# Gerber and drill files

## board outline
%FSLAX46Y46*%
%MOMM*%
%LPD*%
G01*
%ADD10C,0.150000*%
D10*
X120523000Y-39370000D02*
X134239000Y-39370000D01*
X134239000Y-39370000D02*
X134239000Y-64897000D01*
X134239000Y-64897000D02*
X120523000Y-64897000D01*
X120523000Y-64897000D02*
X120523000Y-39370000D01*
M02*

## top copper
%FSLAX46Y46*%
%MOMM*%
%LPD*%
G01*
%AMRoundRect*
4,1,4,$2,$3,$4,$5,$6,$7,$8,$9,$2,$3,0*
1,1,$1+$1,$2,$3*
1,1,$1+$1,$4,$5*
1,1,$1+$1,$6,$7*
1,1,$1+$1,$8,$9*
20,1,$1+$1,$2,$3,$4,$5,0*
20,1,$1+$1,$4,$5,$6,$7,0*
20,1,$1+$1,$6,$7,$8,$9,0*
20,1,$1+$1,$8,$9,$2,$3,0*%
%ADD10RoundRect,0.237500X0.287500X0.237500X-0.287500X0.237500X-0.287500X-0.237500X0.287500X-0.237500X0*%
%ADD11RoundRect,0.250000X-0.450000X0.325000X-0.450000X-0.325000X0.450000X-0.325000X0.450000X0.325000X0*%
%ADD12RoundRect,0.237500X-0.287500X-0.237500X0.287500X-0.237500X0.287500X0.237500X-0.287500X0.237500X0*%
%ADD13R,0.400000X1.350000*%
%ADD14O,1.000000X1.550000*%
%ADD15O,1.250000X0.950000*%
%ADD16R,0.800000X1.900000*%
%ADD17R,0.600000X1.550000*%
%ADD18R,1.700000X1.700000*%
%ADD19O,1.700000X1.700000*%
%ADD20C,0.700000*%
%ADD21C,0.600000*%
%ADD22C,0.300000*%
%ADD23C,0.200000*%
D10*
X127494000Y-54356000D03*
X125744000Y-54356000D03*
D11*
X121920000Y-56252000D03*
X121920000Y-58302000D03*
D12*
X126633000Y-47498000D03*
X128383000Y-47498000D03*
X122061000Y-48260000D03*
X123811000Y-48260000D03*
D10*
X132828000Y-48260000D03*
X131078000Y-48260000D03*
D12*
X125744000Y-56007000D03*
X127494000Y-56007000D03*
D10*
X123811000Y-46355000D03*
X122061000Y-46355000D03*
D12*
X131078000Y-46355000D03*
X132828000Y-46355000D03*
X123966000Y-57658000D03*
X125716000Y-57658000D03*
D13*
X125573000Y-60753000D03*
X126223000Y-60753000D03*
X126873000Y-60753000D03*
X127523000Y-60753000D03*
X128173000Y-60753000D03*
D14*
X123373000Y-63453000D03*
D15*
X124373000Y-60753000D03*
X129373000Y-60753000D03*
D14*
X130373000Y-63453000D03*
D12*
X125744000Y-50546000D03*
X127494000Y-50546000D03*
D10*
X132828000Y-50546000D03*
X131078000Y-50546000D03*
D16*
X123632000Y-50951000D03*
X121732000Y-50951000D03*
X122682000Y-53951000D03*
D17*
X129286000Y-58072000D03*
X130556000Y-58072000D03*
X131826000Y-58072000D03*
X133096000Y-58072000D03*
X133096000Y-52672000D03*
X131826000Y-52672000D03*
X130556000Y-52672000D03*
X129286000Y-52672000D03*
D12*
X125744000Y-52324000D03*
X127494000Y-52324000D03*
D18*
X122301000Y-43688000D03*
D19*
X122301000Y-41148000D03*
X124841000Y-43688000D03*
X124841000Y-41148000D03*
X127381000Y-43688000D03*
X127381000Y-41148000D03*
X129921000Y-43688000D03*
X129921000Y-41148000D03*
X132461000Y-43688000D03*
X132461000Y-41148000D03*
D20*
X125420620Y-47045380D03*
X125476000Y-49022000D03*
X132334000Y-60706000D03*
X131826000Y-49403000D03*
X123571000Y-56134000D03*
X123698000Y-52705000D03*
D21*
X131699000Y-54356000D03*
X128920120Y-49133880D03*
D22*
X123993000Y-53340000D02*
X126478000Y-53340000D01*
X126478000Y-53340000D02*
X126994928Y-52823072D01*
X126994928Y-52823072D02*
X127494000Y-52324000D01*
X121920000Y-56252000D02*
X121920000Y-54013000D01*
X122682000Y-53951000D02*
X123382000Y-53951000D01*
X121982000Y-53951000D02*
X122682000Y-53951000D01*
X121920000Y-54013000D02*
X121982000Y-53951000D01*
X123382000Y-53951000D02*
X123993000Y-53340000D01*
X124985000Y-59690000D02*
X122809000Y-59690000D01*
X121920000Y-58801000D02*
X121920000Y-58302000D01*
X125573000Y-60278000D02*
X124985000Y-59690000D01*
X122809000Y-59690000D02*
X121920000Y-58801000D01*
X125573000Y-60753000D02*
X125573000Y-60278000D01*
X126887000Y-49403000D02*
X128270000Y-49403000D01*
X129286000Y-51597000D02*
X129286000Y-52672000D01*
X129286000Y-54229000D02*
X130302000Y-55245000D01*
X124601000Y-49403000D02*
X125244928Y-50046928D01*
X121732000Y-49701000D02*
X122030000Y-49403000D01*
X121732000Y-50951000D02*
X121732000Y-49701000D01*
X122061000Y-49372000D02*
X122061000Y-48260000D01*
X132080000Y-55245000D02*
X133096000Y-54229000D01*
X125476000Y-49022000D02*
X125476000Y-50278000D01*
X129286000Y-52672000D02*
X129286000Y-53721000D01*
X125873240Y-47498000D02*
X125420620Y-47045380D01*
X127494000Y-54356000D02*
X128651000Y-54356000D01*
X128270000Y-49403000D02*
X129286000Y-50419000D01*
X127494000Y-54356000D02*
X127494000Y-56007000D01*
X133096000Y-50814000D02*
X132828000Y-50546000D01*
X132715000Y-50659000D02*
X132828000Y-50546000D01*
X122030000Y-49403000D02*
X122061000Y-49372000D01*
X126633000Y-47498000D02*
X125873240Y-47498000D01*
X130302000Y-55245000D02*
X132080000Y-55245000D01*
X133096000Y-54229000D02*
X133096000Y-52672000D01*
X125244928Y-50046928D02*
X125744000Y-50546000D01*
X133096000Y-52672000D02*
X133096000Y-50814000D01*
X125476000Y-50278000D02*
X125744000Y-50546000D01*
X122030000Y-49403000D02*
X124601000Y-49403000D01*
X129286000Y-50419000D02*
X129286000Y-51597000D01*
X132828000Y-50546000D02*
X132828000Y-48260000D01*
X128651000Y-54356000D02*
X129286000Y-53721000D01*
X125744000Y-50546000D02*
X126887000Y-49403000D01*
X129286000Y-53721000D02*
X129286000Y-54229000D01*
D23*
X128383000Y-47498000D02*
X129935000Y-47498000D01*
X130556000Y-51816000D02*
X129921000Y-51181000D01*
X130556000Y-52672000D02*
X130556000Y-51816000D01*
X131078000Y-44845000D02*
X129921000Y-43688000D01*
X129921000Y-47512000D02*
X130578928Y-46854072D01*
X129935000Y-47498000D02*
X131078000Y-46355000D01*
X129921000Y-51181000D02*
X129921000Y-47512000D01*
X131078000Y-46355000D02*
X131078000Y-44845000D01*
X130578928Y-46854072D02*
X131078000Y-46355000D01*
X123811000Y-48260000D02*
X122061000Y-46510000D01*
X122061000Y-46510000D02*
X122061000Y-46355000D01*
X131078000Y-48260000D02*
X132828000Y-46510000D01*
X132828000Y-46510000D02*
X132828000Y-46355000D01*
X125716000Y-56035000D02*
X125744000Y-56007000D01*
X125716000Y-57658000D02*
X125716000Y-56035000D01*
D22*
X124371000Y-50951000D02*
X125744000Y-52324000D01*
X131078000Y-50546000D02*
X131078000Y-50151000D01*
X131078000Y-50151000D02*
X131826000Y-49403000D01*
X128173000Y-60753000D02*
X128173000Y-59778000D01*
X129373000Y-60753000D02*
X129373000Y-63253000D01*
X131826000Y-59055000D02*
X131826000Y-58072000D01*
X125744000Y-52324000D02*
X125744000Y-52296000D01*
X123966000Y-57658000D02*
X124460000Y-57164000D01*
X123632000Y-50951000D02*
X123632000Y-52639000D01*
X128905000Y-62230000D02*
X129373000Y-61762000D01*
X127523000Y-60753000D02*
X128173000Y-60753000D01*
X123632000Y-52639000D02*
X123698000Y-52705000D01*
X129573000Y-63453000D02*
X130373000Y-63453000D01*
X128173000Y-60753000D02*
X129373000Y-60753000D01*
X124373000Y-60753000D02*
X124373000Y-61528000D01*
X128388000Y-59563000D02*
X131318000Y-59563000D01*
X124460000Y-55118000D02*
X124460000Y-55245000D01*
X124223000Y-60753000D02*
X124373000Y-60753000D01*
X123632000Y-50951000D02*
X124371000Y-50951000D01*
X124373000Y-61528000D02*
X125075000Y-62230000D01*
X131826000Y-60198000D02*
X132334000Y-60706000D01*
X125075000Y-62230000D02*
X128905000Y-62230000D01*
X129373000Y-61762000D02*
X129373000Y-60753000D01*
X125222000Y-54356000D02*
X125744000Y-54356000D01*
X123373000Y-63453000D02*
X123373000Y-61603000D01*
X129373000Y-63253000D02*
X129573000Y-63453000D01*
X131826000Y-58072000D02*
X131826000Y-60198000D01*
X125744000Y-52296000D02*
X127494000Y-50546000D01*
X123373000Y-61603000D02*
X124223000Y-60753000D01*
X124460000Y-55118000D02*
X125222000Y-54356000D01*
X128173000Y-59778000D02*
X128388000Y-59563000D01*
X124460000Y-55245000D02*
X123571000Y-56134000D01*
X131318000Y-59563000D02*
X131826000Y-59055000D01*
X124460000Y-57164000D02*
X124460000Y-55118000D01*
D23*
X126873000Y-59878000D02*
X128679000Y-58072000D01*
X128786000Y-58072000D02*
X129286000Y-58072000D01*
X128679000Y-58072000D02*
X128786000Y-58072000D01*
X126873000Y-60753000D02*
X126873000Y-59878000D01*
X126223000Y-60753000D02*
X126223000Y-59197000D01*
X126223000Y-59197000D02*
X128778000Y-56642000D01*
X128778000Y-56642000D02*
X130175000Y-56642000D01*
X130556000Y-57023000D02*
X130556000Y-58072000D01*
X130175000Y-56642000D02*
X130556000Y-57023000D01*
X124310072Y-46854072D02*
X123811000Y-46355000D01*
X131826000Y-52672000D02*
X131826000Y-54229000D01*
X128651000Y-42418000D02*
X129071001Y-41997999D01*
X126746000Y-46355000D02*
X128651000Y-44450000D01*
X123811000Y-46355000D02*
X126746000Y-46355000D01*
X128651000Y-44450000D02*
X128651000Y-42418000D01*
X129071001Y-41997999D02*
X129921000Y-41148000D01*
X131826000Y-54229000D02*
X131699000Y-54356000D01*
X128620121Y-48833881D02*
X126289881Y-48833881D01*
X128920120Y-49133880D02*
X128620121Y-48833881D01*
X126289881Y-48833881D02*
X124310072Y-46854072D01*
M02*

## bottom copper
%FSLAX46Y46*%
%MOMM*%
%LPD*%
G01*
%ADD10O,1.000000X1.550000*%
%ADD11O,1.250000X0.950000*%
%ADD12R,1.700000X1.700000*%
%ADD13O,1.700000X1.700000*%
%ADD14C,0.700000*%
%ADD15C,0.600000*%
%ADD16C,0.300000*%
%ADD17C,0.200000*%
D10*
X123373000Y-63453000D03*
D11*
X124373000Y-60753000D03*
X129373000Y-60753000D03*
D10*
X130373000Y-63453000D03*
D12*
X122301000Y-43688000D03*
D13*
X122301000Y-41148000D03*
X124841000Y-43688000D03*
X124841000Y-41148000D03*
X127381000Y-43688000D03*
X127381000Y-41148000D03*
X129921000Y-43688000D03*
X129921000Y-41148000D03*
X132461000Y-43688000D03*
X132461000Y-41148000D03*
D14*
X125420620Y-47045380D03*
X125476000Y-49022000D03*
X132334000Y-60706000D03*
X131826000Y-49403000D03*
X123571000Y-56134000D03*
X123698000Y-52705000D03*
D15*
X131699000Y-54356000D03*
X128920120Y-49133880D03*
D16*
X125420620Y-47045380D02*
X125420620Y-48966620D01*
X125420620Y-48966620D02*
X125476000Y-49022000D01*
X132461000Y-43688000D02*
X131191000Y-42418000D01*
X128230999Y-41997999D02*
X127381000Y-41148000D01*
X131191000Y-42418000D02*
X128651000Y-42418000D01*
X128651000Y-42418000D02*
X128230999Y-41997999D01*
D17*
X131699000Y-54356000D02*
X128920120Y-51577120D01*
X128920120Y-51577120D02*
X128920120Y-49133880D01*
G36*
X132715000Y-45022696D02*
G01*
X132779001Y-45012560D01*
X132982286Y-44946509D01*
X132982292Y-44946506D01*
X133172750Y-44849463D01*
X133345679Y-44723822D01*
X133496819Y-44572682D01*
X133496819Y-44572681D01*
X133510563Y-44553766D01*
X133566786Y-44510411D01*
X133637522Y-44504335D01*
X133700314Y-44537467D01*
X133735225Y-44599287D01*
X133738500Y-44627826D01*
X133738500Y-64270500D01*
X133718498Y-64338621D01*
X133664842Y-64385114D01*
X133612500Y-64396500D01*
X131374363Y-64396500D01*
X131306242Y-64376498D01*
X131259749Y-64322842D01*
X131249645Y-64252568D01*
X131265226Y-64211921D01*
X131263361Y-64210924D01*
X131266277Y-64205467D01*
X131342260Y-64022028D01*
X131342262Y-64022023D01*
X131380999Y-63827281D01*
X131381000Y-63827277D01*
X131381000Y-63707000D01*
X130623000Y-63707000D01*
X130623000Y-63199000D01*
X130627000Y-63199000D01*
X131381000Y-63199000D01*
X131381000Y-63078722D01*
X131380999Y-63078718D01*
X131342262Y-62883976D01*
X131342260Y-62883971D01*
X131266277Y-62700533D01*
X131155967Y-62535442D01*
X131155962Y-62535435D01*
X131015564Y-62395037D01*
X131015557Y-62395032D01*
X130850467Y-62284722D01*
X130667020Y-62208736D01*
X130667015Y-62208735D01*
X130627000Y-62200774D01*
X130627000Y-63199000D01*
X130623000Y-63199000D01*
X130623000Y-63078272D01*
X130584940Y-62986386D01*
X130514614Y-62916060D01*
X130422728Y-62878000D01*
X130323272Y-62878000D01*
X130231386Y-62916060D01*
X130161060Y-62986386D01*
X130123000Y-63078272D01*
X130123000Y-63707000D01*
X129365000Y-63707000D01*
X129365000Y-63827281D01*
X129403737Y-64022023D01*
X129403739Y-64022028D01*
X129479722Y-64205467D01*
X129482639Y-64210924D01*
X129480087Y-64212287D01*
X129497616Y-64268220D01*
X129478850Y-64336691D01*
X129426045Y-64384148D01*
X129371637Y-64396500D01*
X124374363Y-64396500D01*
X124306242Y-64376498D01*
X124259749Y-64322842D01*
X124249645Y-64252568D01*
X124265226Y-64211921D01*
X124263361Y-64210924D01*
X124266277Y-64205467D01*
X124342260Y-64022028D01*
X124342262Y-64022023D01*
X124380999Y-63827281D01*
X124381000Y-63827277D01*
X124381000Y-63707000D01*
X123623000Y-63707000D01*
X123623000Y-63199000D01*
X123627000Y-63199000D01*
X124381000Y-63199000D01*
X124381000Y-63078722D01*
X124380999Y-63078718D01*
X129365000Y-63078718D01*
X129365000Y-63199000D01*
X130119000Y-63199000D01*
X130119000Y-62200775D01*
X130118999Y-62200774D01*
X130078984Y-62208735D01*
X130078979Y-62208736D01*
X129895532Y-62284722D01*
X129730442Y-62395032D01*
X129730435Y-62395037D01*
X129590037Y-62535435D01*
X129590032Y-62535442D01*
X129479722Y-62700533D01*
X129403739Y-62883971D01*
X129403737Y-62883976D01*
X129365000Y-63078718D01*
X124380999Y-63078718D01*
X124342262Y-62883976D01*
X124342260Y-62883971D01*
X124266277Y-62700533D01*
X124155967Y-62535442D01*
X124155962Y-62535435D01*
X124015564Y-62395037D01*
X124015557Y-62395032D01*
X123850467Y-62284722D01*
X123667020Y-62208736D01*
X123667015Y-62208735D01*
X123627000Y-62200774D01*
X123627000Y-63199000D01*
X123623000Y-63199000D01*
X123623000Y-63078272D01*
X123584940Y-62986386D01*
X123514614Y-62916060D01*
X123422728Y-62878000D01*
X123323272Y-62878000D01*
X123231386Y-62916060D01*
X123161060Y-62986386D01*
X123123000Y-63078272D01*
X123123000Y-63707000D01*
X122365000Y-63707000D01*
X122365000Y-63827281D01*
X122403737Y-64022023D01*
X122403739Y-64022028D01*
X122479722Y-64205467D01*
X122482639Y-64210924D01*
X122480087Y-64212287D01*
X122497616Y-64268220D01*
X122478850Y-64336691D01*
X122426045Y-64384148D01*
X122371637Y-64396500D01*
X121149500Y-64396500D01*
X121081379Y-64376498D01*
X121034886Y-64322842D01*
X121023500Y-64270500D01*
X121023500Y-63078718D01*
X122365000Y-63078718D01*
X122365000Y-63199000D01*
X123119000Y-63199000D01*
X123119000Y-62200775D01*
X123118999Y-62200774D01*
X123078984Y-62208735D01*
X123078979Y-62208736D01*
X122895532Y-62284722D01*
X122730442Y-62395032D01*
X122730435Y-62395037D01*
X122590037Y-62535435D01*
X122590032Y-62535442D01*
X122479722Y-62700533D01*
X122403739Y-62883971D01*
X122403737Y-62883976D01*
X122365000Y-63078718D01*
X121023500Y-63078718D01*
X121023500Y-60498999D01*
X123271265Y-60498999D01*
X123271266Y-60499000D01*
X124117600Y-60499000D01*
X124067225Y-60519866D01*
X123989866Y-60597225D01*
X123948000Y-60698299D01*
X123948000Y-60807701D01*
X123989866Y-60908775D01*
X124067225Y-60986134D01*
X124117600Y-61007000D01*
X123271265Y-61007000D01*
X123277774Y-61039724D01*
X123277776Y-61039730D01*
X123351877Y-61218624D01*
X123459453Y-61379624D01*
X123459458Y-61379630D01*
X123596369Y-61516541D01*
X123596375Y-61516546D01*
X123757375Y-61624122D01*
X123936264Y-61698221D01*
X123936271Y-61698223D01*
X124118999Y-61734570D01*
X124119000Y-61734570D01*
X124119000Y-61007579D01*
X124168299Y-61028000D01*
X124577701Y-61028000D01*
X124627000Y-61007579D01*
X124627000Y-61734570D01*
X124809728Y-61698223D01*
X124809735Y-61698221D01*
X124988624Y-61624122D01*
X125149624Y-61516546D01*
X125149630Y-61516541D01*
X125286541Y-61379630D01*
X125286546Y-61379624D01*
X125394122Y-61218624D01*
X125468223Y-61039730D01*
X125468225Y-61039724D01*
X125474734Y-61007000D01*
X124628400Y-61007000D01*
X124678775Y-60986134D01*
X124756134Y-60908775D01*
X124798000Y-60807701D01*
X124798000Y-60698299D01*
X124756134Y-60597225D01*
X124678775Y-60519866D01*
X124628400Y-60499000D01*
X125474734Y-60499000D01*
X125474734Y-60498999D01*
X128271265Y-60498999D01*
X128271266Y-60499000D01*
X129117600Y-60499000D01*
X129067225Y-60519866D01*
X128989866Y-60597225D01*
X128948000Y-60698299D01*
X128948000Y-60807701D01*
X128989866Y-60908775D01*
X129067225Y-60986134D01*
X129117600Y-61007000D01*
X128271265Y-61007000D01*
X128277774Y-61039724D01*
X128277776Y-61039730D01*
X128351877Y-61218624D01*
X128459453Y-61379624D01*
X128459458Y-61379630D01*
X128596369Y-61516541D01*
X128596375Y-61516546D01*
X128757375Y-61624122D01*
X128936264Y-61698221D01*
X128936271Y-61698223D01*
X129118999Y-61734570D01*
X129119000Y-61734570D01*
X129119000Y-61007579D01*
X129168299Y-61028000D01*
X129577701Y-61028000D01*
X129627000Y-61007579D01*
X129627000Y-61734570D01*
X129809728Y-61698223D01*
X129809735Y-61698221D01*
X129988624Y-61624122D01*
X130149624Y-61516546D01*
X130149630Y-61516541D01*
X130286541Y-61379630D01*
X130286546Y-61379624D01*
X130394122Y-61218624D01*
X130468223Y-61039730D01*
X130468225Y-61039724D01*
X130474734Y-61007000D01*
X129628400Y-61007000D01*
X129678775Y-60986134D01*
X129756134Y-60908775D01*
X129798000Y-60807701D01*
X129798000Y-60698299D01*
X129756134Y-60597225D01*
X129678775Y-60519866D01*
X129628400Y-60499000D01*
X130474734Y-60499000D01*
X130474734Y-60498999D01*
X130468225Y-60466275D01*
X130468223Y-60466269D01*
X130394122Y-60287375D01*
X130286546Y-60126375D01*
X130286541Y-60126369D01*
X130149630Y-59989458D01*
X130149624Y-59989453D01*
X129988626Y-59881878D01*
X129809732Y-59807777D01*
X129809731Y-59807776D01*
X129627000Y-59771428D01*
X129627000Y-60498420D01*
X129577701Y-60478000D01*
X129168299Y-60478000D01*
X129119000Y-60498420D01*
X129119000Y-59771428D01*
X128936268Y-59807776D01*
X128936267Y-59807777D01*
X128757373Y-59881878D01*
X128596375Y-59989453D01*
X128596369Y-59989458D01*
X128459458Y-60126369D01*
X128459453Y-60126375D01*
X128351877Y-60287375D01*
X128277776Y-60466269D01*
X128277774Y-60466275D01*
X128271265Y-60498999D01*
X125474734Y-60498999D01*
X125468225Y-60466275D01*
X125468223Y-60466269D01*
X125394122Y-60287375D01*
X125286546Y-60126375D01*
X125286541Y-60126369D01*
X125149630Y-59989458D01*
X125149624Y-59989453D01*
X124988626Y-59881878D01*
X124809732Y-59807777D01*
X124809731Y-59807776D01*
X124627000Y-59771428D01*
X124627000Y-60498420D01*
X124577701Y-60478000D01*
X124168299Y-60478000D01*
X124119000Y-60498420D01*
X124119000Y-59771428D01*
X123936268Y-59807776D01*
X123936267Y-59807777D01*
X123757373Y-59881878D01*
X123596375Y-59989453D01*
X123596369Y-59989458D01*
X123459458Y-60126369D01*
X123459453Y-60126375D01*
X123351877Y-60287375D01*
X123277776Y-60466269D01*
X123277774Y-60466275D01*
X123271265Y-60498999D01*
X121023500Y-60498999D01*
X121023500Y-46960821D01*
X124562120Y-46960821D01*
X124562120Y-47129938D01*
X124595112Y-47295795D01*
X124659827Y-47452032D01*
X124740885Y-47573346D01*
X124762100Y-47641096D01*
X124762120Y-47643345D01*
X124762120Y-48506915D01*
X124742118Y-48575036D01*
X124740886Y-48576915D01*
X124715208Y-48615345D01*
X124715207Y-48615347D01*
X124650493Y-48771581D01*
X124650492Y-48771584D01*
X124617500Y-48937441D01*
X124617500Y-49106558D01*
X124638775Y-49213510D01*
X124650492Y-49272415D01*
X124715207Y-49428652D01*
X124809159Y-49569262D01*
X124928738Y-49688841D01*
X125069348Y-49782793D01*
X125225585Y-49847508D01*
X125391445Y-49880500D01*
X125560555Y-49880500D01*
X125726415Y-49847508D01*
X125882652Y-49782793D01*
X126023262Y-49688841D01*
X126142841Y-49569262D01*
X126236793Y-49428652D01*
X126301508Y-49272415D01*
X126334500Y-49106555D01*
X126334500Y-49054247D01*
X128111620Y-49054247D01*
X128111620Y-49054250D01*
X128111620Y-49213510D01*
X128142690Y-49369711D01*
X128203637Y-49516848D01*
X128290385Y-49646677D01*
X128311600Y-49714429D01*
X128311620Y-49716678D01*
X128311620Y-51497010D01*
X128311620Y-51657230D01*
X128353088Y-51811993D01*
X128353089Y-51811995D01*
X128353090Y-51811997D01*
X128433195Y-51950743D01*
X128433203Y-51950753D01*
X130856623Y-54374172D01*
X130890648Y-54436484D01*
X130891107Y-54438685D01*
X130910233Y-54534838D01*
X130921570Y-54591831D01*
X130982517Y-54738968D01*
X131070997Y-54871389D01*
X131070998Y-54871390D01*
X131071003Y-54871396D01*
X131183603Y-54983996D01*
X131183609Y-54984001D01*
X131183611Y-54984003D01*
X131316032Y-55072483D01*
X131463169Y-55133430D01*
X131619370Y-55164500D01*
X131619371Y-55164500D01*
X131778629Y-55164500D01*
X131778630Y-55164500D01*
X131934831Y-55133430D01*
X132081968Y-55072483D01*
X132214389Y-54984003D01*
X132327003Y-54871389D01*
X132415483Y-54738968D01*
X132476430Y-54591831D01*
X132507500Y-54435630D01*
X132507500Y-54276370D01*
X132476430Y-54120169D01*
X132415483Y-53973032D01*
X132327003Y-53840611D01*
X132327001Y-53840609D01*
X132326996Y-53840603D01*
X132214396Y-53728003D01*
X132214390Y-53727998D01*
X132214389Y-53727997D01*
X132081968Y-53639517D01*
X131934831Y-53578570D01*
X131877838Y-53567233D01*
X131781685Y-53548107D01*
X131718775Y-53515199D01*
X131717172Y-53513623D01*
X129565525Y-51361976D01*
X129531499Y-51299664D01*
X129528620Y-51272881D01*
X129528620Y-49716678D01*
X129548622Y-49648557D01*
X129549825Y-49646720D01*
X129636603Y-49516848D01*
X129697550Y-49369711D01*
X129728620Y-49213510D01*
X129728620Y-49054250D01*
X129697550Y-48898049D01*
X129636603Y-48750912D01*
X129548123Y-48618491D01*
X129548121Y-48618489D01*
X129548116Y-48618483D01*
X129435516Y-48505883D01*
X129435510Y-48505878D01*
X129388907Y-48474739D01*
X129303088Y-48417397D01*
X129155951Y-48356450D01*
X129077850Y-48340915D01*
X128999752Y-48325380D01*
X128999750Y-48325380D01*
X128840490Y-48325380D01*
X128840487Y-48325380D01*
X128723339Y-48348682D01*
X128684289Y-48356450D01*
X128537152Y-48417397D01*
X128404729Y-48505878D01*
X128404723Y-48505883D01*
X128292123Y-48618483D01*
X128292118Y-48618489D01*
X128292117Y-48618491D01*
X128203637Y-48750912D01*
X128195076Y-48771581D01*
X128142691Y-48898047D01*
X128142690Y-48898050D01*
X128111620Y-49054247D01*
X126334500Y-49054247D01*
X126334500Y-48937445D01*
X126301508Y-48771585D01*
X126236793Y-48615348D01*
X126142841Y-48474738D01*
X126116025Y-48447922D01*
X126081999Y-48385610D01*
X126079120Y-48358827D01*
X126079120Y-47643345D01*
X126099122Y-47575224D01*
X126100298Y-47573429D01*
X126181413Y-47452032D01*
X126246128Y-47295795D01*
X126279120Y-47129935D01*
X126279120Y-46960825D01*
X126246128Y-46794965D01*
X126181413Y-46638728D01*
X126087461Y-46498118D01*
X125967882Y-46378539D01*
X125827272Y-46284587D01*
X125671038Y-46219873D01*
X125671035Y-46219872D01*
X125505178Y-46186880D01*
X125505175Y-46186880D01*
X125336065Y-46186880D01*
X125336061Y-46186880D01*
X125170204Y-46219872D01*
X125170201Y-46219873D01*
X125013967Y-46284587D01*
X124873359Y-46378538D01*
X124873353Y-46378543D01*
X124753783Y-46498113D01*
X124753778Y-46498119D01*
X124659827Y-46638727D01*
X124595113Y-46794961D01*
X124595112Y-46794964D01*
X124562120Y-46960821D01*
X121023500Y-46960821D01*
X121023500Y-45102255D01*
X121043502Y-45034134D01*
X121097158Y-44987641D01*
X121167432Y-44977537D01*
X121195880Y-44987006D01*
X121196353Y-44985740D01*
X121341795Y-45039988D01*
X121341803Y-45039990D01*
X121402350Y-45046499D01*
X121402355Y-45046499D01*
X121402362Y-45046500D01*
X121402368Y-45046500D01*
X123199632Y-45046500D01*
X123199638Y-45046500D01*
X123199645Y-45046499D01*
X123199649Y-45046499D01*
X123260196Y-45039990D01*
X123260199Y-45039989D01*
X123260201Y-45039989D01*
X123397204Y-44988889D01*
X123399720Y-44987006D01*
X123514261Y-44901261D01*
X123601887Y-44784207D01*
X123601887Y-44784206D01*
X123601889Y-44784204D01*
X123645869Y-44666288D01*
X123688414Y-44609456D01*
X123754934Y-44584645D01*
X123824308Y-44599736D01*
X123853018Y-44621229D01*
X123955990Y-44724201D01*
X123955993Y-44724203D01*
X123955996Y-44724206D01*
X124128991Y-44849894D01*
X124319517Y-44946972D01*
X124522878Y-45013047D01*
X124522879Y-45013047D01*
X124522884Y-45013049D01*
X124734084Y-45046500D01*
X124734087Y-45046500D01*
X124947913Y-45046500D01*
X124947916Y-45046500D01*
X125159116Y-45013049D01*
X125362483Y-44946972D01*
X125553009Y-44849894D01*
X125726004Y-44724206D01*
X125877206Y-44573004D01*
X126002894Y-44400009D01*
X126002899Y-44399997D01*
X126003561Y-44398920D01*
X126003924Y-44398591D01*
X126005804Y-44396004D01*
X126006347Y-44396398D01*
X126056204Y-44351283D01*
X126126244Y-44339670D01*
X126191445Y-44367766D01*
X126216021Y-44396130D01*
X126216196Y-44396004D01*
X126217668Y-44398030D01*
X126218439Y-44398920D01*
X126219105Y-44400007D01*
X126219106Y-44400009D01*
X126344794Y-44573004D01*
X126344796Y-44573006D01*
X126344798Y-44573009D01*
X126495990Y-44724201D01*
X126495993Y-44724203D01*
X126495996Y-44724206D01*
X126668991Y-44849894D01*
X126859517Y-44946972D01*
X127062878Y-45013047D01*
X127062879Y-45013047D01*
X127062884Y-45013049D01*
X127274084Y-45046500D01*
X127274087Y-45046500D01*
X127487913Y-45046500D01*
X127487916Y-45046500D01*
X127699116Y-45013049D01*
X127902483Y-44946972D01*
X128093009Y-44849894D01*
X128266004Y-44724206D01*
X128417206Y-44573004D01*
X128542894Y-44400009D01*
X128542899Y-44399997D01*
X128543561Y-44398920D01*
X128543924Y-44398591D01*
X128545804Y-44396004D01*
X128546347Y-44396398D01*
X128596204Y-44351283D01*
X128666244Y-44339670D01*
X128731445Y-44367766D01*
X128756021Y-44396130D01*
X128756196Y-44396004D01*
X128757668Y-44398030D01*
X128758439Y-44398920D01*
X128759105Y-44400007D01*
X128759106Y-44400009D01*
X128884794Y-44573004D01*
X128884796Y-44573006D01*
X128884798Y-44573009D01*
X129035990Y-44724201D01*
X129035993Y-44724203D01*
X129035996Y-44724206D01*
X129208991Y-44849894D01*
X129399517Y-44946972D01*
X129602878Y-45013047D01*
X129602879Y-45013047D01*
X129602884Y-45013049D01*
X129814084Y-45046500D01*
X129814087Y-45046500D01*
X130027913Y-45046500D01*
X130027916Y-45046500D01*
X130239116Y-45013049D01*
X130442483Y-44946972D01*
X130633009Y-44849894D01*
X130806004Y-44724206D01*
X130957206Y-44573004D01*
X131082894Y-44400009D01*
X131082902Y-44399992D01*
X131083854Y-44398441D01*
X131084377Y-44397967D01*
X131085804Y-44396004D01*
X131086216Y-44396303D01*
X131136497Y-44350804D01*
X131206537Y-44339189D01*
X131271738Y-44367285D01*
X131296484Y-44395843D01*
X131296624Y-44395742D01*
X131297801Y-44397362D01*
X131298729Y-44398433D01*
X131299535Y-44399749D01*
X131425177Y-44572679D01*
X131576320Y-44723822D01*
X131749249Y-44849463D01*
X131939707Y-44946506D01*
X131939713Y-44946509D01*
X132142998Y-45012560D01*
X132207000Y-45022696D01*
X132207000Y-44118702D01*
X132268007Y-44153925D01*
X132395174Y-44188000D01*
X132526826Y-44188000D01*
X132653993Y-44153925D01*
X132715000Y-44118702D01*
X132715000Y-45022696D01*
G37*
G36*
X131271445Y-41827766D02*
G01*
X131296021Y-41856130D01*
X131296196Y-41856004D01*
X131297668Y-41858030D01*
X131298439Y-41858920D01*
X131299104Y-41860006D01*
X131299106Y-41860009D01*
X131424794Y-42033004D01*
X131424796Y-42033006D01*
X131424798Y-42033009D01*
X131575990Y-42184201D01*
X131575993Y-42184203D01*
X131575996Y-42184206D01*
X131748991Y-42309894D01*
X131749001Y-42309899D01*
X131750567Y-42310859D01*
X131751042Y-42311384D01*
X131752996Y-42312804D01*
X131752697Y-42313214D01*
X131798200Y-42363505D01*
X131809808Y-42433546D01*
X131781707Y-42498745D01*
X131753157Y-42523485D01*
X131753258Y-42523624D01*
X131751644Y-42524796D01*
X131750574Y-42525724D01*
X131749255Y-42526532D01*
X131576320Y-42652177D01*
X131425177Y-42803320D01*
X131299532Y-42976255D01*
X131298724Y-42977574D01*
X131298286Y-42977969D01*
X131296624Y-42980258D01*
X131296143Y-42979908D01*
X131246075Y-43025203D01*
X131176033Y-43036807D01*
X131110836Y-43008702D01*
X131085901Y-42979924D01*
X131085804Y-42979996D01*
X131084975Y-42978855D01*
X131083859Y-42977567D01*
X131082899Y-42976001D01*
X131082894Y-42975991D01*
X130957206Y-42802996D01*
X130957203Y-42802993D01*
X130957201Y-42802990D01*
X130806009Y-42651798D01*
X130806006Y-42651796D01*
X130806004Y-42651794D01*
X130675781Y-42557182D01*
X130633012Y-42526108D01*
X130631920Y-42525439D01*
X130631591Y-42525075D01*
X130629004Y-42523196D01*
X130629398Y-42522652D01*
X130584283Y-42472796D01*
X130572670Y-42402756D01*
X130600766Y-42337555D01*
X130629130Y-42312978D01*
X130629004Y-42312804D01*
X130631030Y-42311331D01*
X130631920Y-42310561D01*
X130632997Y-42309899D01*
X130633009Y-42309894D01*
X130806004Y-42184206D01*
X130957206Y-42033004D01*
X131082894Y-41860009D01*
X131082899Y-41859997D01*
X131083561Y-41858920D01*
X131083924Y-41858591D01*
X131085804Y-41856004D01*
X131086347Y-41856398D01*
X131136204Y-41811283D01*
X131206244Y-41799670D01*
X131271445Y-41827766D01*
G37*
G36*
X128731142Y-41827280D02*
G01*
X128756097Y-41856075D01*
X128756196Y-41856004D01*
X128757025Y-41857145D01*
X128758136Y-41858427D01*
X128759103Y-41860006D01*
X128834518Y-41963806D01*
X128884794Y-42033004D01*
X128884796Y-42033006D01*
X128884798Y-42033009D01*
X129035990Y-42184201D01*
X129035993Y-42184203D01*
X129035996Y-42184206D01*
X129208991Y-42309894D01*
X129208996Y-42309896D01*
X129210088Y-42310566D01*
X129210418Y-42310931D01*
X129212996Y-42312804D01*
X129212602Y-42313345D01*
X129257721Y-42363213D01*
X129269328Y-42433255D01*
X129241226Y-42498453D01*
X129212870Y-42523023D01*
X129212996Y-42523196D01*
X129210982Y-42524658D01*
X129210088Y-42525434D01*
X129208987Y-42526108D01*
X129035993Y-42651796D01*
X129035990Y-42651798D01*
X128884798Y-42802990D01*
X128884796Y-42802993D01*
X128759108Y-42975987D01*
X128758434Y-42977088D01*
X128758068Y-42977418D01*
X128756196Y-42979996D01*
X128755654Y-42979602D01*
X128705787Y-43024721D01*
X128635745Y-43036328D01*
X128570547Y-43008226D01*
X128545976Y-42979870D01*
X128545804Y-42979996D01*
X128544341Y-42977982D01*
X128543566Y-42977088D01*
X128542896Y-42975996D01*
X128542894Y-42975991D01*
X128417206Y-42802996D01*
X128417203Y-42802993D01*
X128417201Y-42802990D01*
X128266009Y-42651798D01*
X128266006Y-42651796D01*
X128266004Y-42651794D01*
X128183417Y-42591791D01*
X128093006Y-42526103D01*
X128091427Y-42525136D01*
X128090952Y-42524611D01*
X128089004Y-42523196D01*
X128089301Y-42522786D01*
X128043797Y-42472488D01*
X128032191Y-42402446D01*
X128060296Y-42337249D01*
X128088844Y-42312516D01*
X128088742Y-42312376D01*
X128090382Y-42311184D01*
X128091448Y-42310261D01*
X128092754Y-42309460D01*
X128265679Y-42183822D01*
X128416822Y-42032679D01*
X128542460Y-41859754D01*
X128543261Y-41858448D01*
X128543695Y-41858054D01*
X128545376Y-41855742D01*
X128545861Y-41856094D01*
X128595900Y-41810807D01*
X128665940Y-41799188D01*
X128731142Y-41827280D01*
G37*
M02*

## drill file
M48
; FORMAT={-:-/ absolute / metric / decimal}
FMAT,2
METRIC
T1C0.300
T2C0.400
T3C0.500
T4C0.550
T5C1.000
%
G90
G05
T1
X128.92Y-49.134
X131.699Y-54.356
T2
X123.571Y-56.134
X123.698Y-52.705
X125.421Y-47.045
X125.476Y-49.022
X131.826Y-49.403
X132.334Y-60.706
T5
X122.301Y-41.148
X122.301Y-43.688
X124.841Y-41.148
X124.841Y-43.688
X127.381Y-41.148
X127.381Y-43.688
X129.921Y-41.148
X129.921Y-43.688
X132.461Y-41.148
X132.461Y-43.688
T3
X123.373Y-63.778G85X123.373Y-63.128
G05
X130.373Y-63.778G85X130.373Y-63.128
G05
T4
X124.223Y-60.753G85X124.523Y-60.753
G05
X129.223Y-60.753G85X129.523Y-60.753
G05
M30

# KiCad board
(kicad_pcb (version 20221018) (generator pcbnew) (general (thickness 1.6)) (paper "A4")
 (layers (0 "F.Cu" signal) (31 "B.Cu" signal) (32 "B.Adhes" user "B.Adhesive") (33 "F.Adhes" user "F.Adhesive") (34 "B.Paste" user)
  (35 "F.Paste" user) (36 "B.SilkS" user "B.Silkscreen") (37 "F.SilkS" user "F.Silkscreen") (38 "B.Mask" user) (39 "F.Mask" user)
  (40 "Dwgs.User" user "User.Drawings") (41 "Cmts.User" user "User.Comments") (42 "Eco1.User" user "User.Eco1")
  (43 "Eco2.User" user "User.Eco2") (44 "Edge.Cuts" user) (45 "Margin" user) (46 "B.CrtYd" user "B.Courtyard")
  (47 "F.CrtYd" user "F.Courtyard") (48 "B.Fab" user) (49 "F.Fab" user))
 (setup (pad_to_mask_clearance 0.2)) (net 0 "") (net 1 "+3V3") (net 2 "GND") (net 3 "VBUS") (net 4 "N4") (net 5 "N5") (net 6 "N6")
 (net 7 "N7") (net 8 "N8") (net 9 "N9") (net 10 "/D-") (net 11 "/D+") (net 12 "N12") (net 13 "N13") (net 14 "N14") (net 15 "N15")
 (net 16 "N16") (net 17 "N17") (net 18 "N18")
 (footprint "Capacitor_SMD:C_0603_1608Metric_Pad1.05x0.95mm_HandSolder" (layer "F.Cu") (at 126.619 54.356 180)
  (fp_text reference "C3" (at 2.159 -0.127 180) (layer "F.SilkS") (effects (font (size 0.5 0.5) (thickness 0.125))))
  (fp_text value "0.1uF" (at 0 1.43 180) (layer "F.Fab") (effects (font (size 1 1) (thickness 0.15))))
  (pad "1" smd roundrect (at -0.875 0 180) (size 1.05 0.95) (layers "F.Cu" "F.Paste" "F.Mask") (roundrect_rratio 0.25) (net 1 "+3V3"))
  (pad "2" smd roundrect (at 0.875 0 180) (size 1.05 0.95) (layers "F.Cu" "F.Paste" "F.Mask") (roundrect_rratio 0.25) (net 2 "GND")))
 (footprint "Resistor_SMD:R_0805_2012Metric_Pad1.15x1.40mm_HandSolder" (layer "F.Cu") (at 121.92 57.277 -90)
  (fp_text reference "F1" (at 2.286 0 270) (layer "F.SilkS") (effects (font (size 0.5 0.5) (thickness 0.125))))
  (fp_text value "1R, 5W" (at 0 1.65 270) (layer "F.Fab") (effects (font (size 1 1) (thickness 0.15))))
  (pad "1" smd roundrect (at -1.025 0 270) (size 1.15 1.4) (layers "F.Cu" "F.Paste" "F.Mask") (roundrect_rratio 0.217391) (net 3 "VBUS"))
  (pad "2" smd roundrect (at 1.025 0 270) (size 1.15 1.4) (layers "F.Cu" "F.Paste" "F.Mask") (roundrect_rratio 0.217391) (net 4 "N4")))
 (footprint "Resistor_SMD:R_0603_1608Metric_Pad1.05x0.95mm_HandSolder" (layer "F.Cu") (at 127.508 47.498)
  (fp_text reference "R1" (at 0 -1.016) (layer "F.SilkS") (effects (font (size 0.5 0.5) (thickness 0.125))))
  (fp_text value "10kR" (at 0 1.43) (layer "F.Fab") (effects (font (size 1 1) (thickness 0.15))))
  (pad "1" smd roundrect (at -0.875 0) (size 1.05 0.95) (layers "F.Cu" "F.Paste" "F.Mask") (roundrect_rratio 0.25) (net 1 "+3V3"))
  (pad "2" smd roundrect (at 0.875 0) (size 1.05 0.95) (layers "F.Cu" "F.Paste" "F.Mask") (roundrect_rratio 0.25) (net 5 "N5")))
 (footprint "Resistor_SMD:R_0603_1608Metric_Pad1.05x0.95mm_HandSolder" (layer "F.Cu") (at 122.936 48.26)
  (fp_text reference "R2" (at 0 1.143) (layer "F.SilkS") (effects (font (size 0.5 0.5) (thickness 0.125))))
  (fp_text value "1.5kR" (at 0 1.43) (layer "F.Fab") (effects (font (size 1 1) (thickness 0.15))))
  (pad "1" smd roundrect (at -0.875 0) (size 1.05 0.95) (layers "F.Cu" "F.Paste" "F.Mask") (roundrect_rratio 0.25) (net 1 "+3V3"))
  (pad "2" smd roundrect (at 0.875 0) (size 1.05 0.95) (layers "F.Cu" "F.Paste" "F.Mask") (roundrect_rratio 0.25) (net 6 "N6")))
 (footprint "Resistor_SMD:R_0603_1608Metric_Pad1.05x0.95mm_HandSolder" (layer "F.Cu") (at 131.953 48.26 180)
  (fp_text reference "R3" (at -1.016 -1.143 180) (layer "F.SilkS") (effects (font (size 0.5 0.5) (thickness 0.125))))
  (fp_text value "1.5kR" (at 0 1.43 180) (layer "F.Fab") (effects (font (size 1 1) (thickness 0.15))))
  (pad "1" smd roundrect (at -0.875 0 180) (size 1.05 0.95) (layers "F.Cu" "F.Paste" "F.Mask") (roundrect_rratio 0.25) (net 1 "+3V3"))
  (pad "2" smd roundrect (at 0.875 0 180) (size 1.05 0.95) (layers "F.Cu" "F.Paste" "F.Mask") (roundrect_rratio 0.25) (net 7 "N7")))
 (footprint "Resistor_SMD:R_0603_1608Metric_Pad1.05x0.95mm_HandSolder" (layer "F.Cu") (at 126.619 56.007)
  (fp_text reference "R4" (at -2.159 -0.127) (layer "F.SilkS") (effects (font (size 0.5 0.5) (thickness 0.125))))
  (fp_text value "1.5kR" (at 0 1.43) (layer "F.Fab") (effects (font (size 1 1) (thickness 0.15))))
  (pad "1" smd roundrect (at -0.875 0) (size 1.05 0.95) (layers "F.Cu" "F.Paste" "F.Mask") (roundrect_rratio 0.25) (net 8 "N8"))
  (pad "2" smd roundrect (at 0.875 0) (size 1.05 0.95) (layers "F.Cu" "F.Paste" "F.Mask") (roundrect_rratio 0.25) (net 1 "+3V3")))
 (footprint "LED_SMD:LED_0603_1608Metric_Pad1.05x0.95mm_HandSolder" (layer "F.Cu") (at 122.936 46.355 180)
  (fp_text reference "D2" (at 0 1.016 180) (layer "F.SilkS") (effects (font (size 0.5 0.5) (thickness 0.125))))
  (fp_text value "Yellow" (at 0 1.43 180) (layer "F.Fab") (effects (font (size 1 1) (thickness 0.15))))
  (pad "1" smd roundrect (at -0.875 0 180) (size 1.05 0.95) (layers "F.Cu" "F.Paste" "F.Mask") (roundrect_rratio 0.25) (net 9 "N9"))
  (pad "2" smd roundrect (at 0.875 0 180) (size 1.05 0.95) (layers "F.Cu" "F.Paste" "F.Mask") (roundrect_rratio 0.25) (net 6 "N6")))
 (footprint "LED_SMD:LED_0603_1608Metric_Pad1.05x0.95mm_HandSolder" (layer "F.Cu") (at 131.953 46.355)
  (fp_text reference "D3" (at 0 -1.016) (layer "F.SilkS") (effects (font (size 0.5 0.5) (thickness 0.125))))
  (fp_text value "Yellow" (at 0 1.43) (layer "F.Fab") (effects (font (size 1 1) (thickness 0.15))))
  (pad "1" smd roundrect (at -0.875 0) (size 1.05 0.95) (layers "F.Cu" "F.Paste" "F.Mask") (roundrect_rratio 0.25) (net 5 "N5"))
  (pad "2" smd roundrect (at 0.875 0) (size 1.05 0.95) (layers "F.Cu" "F.Paste" "F.Mask") (roundrect_rratio 0.25) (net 7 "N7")))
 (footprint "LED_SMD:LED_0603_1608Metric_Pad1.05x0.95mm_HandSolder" (layer "F.Cu") (at 124.841 57.658)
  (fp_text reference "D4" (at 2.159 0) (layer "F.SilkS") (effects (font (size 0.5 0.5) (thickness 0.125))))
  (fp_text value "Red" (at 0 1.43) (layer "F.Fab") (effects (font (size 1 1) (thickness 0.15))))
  (pad "1" smd roundrect (at -0.875 0) (size 1.05 0.95) (layers "F.Cu" "F.Paste" "F.Mask") (roundrect_rratio 0.25) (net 2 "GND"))
  (pad "2" smd roundrect (at 0.875 0) (size 1.05 0.95) (layers "F.Cu" "F.Paste" "F.Mask") (roundrect_rratio 0.25) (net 8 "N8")))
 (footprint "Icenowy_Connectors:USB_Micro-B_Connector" (layer "F.Cu") (at 126.873 62.103)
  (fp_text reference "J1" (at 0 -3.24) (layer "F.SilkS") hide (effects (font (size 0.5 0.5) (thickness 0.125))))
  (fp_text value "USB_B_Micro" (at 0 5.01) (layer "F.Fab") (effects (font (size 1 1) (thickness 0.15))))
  (pad "1" smd rect (at -1.3 -1.35 90) (size 1.35 0.4) (layers "F.Cu" "F.Paste" "F.Mask") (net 4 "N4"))
  (pad "2" smd rect (at -0.65 -1.35 90) (size 1.35 0.4) (layers "F.Cu" "F.Paste" "F.Mask") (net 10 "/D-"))
  (pad "3" smd rect (at 0 -1.35 90) (size 1.35 0.4) (layers "F.Cu" "F.Paste" "F.Mask") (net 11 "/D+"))
  (pad "4" smd rect (at 0.65 -1.35 90) (size 1.35 0.4) (layers "F.Cu" "F.Paste" "F.Mask") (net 2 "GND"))
  (pad "5" smd rect (at 1.3 -1.35 90) (size 1.35 0.4) (layers "F.Cu" "F.Paste" "F.Mask") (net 2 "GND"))
  (pad "6" thru_hole oval (at -3.5 1.35 90) (size 1.55 1) (drill oval 1.15 0.5) (layers "*.Cu" "*.Mask") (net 2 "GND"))
  (pad "6" thru_hole oval (at -2.5 -1.35 90) (size 0.95 1.25) (drill oval 0.55 0.85) (layers "*.Cu" "*.Mask") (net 2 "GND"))
  (pad "6" thru_hole oval (at 2.5 -1.35 90) (size 0.95 1.25) (drill oval 0.55 0.85) (layers "*.Cu" "*.Mask") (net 2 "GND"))
  (pad "6" thru_hole oval (at 3.5 1.35 90) (size 1.55 1) (drill oval 1.15 0.5) (layers "*.Cu" "*.Mask") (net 2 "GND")))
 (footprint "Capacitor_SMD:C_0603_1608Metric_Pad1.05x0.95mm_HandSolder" (layer "F.Cu") (at 126.619 50.546)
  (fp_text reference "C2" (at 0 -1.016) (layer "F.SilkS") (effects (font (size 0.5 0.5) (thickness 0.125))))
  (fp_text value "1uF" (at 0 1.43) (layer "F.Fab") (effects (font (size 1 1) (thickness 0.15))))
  (pad "1" smd roundrect (at -0.875 0) (size 1.05 0.95) (layers "F.Cu" "F.Paste" "F.Mask") (roundrect_rratio 0.25) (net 1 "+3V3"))
  (pad "2" smd roundrect (at 0.875 0) (size 1.05 0.95) (layers "F.Cu" "F.Paste" "F.Mask") (roundrect_rratio 0.25) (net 2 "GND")))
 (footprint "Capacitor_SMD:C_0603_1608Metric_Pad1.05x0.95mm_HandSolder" (layer "F.Cu") (at 131.953 50.546 180)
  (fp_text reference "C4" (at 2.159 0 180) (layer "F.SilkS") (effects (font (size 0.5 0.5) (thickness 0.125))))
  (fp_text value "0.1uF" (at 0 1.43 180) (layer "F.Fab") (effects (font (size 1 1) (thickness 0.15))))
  (pad "1" smd roundrect (at -0.875 0 180) (size 1.05 0.95) (layers "F.Cu" "F.Paste" "F.Mask") (roundrect_rratio 0.25) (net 1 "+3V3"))
  (pad "2" smd roundrect (at 0.875 0 180) (size 1.05 0.95) (layers "F.Cu" "F.Paste" "F.Mask") (roundrect_rratio 0.25) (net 2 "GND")))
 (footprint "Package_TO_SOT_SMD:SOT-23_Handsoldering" (layer "F.Cu") (at 122.682 52.451 -90)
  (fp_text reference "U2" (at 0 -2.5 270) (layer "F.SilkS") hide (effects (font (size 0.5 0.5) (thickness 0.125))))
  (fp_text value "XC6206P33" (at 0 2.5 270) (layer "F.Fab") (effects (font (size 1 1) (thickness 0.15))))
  (pad "1" smd rect (at -1.5 -0.95 270) (size 1.9 0.8) (layers "F.Cu" "F.Paste" "F.Mask") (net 2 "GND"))
  (pad "2" smd rect (at -1.5 0.95 270) (size 1.9 0.8) (layers "F.Cu" "F.Paste" "F.Mask") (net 1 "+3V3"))
  (pad "3" smd rect (at 1.5 0 270) (size 1.9 0.8) (layers "F.Cu" "F.Paste" "F.Mask") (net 3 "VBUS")))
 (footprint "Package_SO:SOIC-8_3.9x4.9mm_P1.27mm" (layer "F.Cu") (at 131.191 55.372 90)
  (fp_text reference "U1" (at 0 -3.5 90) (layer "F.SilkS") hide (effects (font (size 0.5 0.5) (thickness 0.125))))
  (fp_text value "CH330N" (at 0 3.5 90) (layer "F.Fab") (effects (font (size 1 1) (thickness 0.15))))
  (pad "1" smd rect (at -2.7 -1.905 90) (size 1.55 0.6) (layers "F.Cu" "F.Paste" "F.Mask") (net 11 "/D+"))
  (pad "2" smd rect (at -2.7 -0.635 90) (size 1.55 0.6) (layers "F.Cu" "F.Paste" "F.Mask") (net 10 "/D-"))
  (pad "3" smd rect (at -2.7 0.635 90) (size 1.55 0.6) (layers "F.Cu" "F.Paste" "F.Mask") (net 2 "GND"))
  (pad "4" smd rect (at -2.7 1.905 90) (size 1.55 0.6) (layers "F.Cu" "F.Paste" "F.Mask") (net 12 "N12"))
  (pad "5" smd rect (at 2.7 1.905 90) (size 1.55 0.6) (layers "F.Cu" "F.Paste" "F.Mask") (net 1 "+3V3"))
  (pad "6" smd rect (at 2.7 0.635 90) (size 1.55 0.6) (layers "F.Cu" "F.Paste" "F.Mask") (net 9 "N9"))
  (pad "7" smd rect (at 2.7 -0.635 90) (size 1.55 0.6) (layers "F.Cu" "F.Paste" "F.Mask") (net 5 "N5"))
  (pad "8" smd rect (at 2.7 -1.905 90) (size 1.55 0.6) (layers "F.Cu" "F.Paste" "F.Mask") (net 1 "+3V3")))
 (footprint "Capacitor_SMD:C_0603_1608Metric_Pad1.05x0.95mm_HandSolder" (layer "F.Cu") (at 126.619 52.324)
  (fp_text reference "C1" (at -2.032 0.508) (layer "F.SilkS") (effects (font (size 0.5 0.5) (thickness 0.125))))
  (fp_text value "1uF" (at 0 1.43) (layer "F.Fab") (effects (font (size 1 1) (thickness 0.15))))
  (pad "1" smd roundrect (at -0.875 0) (size 1.05 0.95) (layers "F.Cu" "F.Paste" "F.Mask") (roundrect_rratio 0.25) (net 2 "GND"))
  (pad "2" smd roundrect (at 0.875 0) (size 1.05 0.95) (layers "F.Cu" "F.Paste" "F.Mask") (roundrect_rratio 0.25) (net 3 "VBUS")))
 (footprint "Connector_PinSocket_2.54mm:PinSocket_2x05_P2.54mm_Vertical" (layer "B.Cu") (at 122.301 43.688 -90)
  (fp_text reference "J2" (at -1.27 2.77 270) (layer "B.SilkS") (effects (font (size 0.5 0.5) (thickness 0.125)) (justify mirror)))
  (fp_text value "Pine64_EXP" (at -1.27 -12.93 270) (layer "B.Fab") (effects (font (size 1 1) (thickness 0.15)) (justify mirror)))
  (pad "1" thru_hole rect (at 0 0 270) (size 1.7 1.7) (drill 1) (layers "*.Cu" "*.Mask") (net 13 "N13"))
  (pad "2" thru_hole oval (at -2.54 0 270) (size 1.7 1.7) (drill 1) (layers "*.Cu" "*.Mask") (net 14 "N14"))
  (pad "3" thru_hole oval (at 0 -2.54 270) (size 1.7 1.7) (drill 1) (layers "*.Cu" "*.Mask") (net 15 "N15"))
  (pad "4" thru_hole oval (at -2.54 -2.54 270) (size 1.7 1.7) (drill 1) (layers "*.Cu" "*.Mask") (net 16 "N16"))
  (pad "5" thru_hole oval (at 0 -5.08 270) (size 1.7 1.7) (drill 1) (layers "*.Cu" "*.Mask") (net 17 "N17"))
  (pad "6" thru_hole oval (at -2.54 -5.08 270) (size 1.7 1.7) (drill 1) (layers "*.Cu" "*.Mask") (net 2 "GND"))
  (pad "7" thru_hole oval (at 0 -7.62 270) (size 1.7 1.7) (drill 1) (layers "*.Cu" "*.Mask") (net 5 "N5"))
  (pad "8" thru_hole oval (at -2.54 -7.62 270) (size 1.7 1.7) (drill 1) (layers "*.Cu" "*.Mask") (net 9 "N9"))
  (pad "9" thru_hole oval (at 0 -10.16 270) (size 1.7 1.7) (drill 1) (layers "*.Cu" "*.Mask") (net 2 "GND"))
  (pad "10" thru_hole oval (at -2.54 -10.16 270) (size 1.7 1.7) (drill 1) (layers "*.Cu" "*.Mask") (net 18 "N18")))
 (gr_line (start 120.523 39.37) (end 134.239 39.37) (stroke (width 0.15) (type solid)) (layer "Edge.Cuts"))
 (gr_line (start 134.239 39.37) (end 134.239 64.897) (stroke (width 0.15) (type solid)) (layer "Edge.Cuts"))
 (gr_line (start 134.239 64.897) (end 120.523 64.897) (stroke (width 0.15) (type solid)) (layer "Edge.Cuts"))
 (gr_line (start 120.523 64.897) (end 120.523 39.37) (stroke (width 0.15) (type solid)) (layer "Edge.Cuts"))
 (segment (start 123.993 53.34) (end 126.478 53.34) (width 0.3) (layer "F.Cu") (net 3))
 (segment (start 126.478 53.34) (end 126.994928 52.823072) (width 0.3) (layer "F.Cu") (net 3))
 (segment (start 126.994928 52.823072) (end 127.494 52.324) (width 0.3) (layer "F.Cu") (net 3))
 (segment (start 121.92 56.252) (end 121.92 54.013) (width 0.3) (layer "F.Cu") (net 3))
 (segment (start 122.682 53.951) (end 123.382 53.951) (width 0.3) (layer "F.Cu") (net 3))
 (segment (start 121.982 53.951) (end 122.682 53.951) (width 0.3) (layer "F.Cu") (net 3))
 (segment (start 121.92 54.013) (end 121.982 53.951) (width 0.3) (layer "F.Cu") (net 3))
 (segment (start 123.382 53.951) (end 123.993 53.34) (width 0.3) (layer "F.Cu") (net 3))
 (segment (start 124.985 59.69) (end 122.809 59.69) (width 0.3) (layer "F.Cu") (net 4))
 (segment (start 121.92 58.801) (end 121.92 58.302) (width 0.3) (layer "F.Cu") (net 4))
 (segment (start 125.573 60.278) (end 124.985 59.69) (width 0.3) (layer "F.Cu") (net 4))
 (segment (start 122.809 59.69) (end 121.92 58.801) (width 0.3) (layer "F.Cu") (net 4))
 (segment (start 125.573 60.753) (end 125.573 60.278) (width 0.3) (layer "F.Cu") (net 4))
 (segment (start 126.887 49.403) (end 128.27 49.403) (width 0.3) (layer "F.Cu") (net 1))
 (segment (start 129.286 51.597) (end 129.286 52.672) (width 0.3) (layer "F.Cu") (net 1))
 (segment (start 129.286 54.229) (end 130.302 55.245) (width 0.3) (layer "F.Cu") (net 1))
 (segment (start 124.601 49.403) (end 125.244928 50.046928) (width 0.3) (layer "F.Cu") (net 1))
 (segment (start 121.732 49.701) (end 122.03 49.403) (width 0.3) (layer "F.Cu") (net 1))
 (segment (start 121.732 50.951) (end 121.732 49.701) (width 0.3) (layer "F.Cu") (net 1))
 (segment (start 122.061 49.372) (end 122.061 48.26) (width 0.3) (layer "F.Cu") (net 1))
 (segment (start 132.08 55.245) (end 133.096 54.229) (width 0.3) (layer "F.Cu") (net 1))
 (segment (start 125.476 49.022) (end 125.476 50.278) (width 0.3) (layer "F.Cu") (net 1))
 (segment (start 129.286 52.672) (end 129.286 53.721) (width 0.3) (layer "F.Cu") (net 1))
 (segment (start 125.87324 47.498) (end 125.42062 47.04538) (width 0.3) (layer "F.Cu") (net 1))
 (segment (start 127.494 54.356) (end 128.651 54.356) (width 0.3) (layer "F.Cu") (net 1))
 (segment (start 128.27 49.403) (end 129.286 50.419) (width 0.3) (layer "F.Cu") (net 1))
 (segment (start 127.494 54.356) (end 127.494 56.007) (width 0.3) (layer "F.Cu") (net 1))
 (segment (start 133.096 50.814) (end 132.828 50.546) (width 0.3) (layer "F.Cu") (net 1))
 (segment (start 132.715 50.659) (end 132.828 50.546) (width 0.3) (layer "F.Cu") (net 1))
 (segment (start 122.03 49.403) (end 122.061 49.372) (width 0.3) (layer "F.Cu") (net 1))
 (segment (start 126.633 47.498) (end 125.87324 47.498) (width 0.3) (layer "F.Cu") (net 1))
 (segment (start 130.302 55.245) (end 132.08 55.245) (width 0.3) (layer "F.Cu") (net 1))
 (segment (start 133.096 54.229) (end 133.096 52.672) (width 0.3) (layer "F.Cu") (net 1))
 (segment (start 125.244928 50.046928) (end 125.744 50.546) (width 0.3) (layer "F.Cu") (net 1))
 (segment (start 133.096 52.672) (end 133.096 50.814) (width 0.3) (layer "F.Cu") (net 1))
 (segment (start 125.476 50.278) (end 125.744 50.546) (width 0.3) (layer "F.Cu") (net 1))
 (segment (start 122.03 49.403) (end 124.601 49.403) (width 0.3) (layer "F.Cu") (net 1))
 (segment (start 129.286 50.419) (end 129.286 51.597) (width 0.3) (layer "F.Cu") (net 1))
 (segment (start 132.828 50.546) (end 132.828 48.26) (width 0.3) (layer "F.Cu") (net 1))
 (segment (start 128.651 54.356) (end 129.286 53.721) (width 0.3) (layer "F.Cu") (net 1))
 (segment (start 125.744 50.546) (end 126.887 49.403) (width 0.3) (layer "F.Cu") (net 1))
 (segment (start 129.286 53.721) (end 129.286 54.229) (width 0.3) (layer "F.Cu") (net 1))
 (via (at 125.42062 47.04538) (size 0.7) (drill 0.4) (layers "F.Cu" "B.Cu") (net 1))
 (via (at 125.476 49.022) (size 0.7) (drill 0.4) (layers "F.Cu" "B.Cu") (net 1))
 (segment (start 125.42062 47.04538) (end 125.42062 48.96662) (width 0.3) (layer "B.Cu") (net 1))
 (segment (start 125.42062 48.96662) (end 125.476 49.022) (width 0.3) (layer "B.Cu") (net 1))
 (segment (start 128.383 47.498) (end 129.935 47.498) (width 0.2) (layer "F.Cu") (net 5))
 (segment (start 130.556 51.816) (end 129.921 51.181) (width 0.2) (layer "F.Cu") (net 5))
 (segment (start 130.556 52.672) (end 130.556 51.816) (width 0.2) (layer "F.Cu") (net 5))
 (segment (start 131.078 44.845) (end 129.921 43.688) (width 0.2) (layer "F.Cu") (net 5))
 (segment (start 129.921 47.512) (end 130.578928 46.854072) (width 0.2) (layer "F.Cu") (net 5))
 (segment (start 129.935 47.498) (end 131.078 46.355) (width 0.2) (layer "F.Cu") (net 5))
 (segment (start 129.921 51.181) (end 129.921 47.512) (width 0.2) (layer "F.Cu") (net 5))
 (segment (start 131.078 46.355) (end 131.078 44.845) (width 0.2) (layer "F.Cu") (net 5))
 (segment (start 130.578928 46.854072) (end 131.078 46.355) (width 0.2) (layer "F.Cu") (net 5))
 (segment (start 123.811 48.26) (end 122.061 46.51) (width 0.2) (layer "F.Cu") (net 6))
 (segment (start 122.061 46.51) (end 122.061 46.355) (width 0.2) (layer "F.Cu") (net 6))
 (segment (start 131.078 48.26) (end 132.828 46.51) (width 0.2) (layer "F.Cu") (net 7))
 (segment (start 132.828 46.51) (end 132.828 46.355) (width 0.2) (layer "F.Cu") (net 7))
 (segment (start 125.716 56.035) (end 125.744 56.007) (width 0.2) (layer "F.Cu") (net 8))
 (segment (start 125.716 57.658) (end 125.716 56.035) (width 0.2) (layer "F.Cu") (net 8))
 (segment (start 124.371 50.951) (end 125.744 52.324) (width 0.3) (layer "F.Cu") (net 2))
 (segment (start 131.078 50.546) (end 131.078 50.151) (width 0.3) (layer "F.Cu") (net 2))
 (segment (start 131.078 50.151) (end 131.826 49.403) (width 0.3) (layer "F.Cu") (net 2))
 (segment (start 128.173 60.753) (end 128.173 59.778) (width 0.3) (layer "F.Cu") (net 2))
 (segment (start 129.373 60.753) (end 129.373 63.253) (width 0.3) (layer "F.Cu") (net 2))
 (segment (start 131.826 59.055) (end 131.826 58.072) (width 0.3) (layer "F.Cu") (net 2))
 (segment (start 125.744 52.324) (end 125.744 52.296) (width 0.3) (layer "F.Cu") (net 2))
 (segment (start 123.966 57.658) (end 124.46 57.164) (width 0.3) (layer "F.Cu") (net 2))
 (segment (start 123.632 50.951) (end 123.632 52.639) (width 0.3) (layer "F.Cu") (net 2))
 (segment (start 128.905 62.23) (end 129.373 61.762) (width 0.3) (layer "F.Cu") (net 2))
 (segment (start 127.523 60.753) (end 128.173 60.753) (width 0.3) (layer "F.Cu") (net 2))
 (segment (start 123.632 52.639) (end 123.698 52.705) (width 0.3) (layer "F.Cu") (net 2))
 (segment (start 129.573 63.453) (end 130.373 63.453) (width 0.3) (layer "F.Cu") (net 2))
 (segment (start 128.173 60.753) (end 129.373 60.753) (width 0.3) (layer "F.Cu") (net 2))
 (segment (start 124.373 60.753) (end 124.373 61.528) (width 0.3) (layer "F.Cu") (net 2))
 (segment (start 128.388 59.563) (end 131.318 59.563) (width 0.3) (layer "F.Cu") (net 2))
 (segment (start 124.46 55.118) (end 124.46 55.245) (width 0.3) (layer "F.Cu") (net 2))
 (segment (start 124.223 60.753) (end 124.373 60.753) (width 0.3) (layer "F.Cu") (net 2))
 (segment (start 123.632 50.951) (end 124.371 50.951) (width 0.3) (layer "F.Cu") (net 2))
 (segment (start 124.373 61.528) (end 125.075 62.23) (width 0.3) (layer "F.Cu") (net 2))
 (segment (start 131.826 60.198) (end 132.334 60.706) (width 0.3) (layer "F.Cu") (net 2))
 (segment (start 125.075 62.23) (end 128.905 62.23) (width 0.3) (layer "F.Cu") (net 2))
 (segment (start 129.373 61.762) (end 129.373 60.753) (width 0.3) (layer "F.Cu") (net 2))
 (segment (start 125.222 54.356) (end 125.744 54.356) (width 0.3) (layer "F.Cu") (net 2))
 (segment (start 123.373 63.453) (end 123.373 61.603) (width 0.3) (layer "F.Cu") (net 2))
 (segment (start 129.373 63.253) (end 129.573 63.453) (width 0.3) (layer "F.Cu") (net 2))
 (segment (start 131.826 58.072) (end 131.826 60.198) (width 0.3) (layer "F.Cu") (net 2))
 (segment (start 125.744 52.296) (end 127.494 50.546) (width 0.3) (layer "F.Cu") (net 2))
 (segment (start 123.373 61.603) (end 124.223 60.753) (width 0.3) (layer "F.Cu") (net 2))
 (segment (start 124.46 55.118) (end 125.222 54.356) (width 0.3) (layer "F.Cu") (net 2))
 (segment (start 128.173 59.778) (end 128.388 59.563) (width 0.3) (layer "F.Cu") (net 2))
 (segment (start 124.46 55.245) (end 123.571 56.134) (width 0.3) (layer "F.Cu") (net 2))
 (segment (start 131.318 59.563) (end 131.826 59.055) (width 0.3) (layer "F.Cu") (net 2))
 (segment (start 124.46 57.164) (end 124.46 55.118) (width 0.3) (layer "F.Cu") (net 2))
 (via (at 132.334 60.706) (size 0.7) (drill 0.4) (layers "F.Cu" "B.Cu") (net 2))
 (via (at 131.826 49.403) (size 0.7) (drill 0.4) (layers "F.Cu" "B.Cu") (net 2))
 (via (at 123.571 56.134) (size 0.7) (drill 0.4) (layers "F.Cu" "B.Cu") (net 2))
 (via (at 123.698 52.705) (size 0.7) (drill 0.4) (layers "F.Cu" "B.Cu") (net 2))
 (segment (start 132.461 43.688) (end 131.191 42.418) (width 0.3) (layer "B.Cu") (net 2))
 (segment (start 128.230999 41.997999) (end 127.381 41.148) (width 0.3) (layer "B.Cu") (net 2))
 (segment (start 131.191 42.418) (end 128.651 42.418) (width 0.3) (layer "B.Cu") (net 2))
 (segment (start 128.651 42.418) (end 128.230999 41.997999) (width 0.3) (layer "B.Cu") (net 2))
 (segment (start 126.873 59.878) (end 128.679 58.072) (width 0.2) (layer "F.Cu") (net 11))
 (segment (start 128.786 58.072) (end 129.286 58.072) (width 0.2) (layer "F.Cu") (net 11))
 (segment (start 128.679 58.072) (end 128.786 58.072) (width 0.2) (layer "F.Cu") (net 11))
 (segment (start 126.873 60.753) (end 126.873 59.878) (width 0.2) (layer "F.Cu") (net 11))
 (segment (start 126.223 60.753) (end 126.223 59.197) (width 0.2) (layer "F.Cu") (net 10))
 (segment (start 126.223 59.197) (end 128.778 56.642) (width 0.2) (layer "F.Cu") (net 10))
 (segment (start 128.778 56.642) (end 130.175 56.642) (width 0.2) (layer "F.Cu") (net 10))
 (segment (start 130.556 57.023) (end 130.556 58.072) (width 0.2) (layer "F.Cu") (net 10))
 (segment (start 130.175 56.642) (end 130.556 57.023) (width 0.2) (layer "F.Cu") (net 10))
 (segment (start 124.310072 46.854072) (end 123.811 46.355) (width 0.2) (layer "F.Cu") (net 9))
 (segment (start 131.826 52.672) (end 131.826 54.229) (width 0.2) (layer "F.Cu") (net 9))
 (segment (start 128.651 42.418) (end 129.071001 41.997999) (width 0.2) (layer "F.Cu") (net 9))
 (segment (start 126.746 46.355) (end 128.651 44.45) (width 0.2) (layer "F.Cu") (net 9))
 (segment (start 123.811 46.355) (end 126.746 46.355) (width 0.2) (layer "F.Cu") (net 9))
 (segment (start 128.651 44.45) (end 128.651 42.418) (width 0.2) (layer "F.Cu") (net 9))
 (segment (start 129.071001 41.997999) (end 129.921 41.148) (width 0.2) (layer "F.Cu") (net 9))
 (segment (start 131.826 54.229) (end 131.699 54.356) (width 0.2) (layer "F.Cu") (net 9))
 (segment (start 128.620121 48.833881) (end 126.289881 48.833881) (width 0.2) (layer "F.Cu") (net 9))
 (segment (start 128.92012 49.13388) (end 128.620121 48.833881) (width 0.2) (layer "F.Cu") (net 9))
 (segment (start 126.289881 48.833881) (end 124.310072 46.854072) (width 0.2) (layer "F.Cu") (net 9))
 (via (at 131.699 54.356) (size 0.6) (drill 0.3) (layers "F.Cu" "B.Cu") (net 9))
 (via (at 128.92012 49.13388) (size 0.6) (drill 0.3) (layers "F.Cu" "B.Cu") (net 9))
 (segment (start 131.699 54.356) (end 128.92012 51.57712) (width 0.2) (layer "B.Cu") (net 9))
 (segment (start 128.92012 51.57712) (end 128.92012 49.13388) (width 0.2) (layer "B.Cu") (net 9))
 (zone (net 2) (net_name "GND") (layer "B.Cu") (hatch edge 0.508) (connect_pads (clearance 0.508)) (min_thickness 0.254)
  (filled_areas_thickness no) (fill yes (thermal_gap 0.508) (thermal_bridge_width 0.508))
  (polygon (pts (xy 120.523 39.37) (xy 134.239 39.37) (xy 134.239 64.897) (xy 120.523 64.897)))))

